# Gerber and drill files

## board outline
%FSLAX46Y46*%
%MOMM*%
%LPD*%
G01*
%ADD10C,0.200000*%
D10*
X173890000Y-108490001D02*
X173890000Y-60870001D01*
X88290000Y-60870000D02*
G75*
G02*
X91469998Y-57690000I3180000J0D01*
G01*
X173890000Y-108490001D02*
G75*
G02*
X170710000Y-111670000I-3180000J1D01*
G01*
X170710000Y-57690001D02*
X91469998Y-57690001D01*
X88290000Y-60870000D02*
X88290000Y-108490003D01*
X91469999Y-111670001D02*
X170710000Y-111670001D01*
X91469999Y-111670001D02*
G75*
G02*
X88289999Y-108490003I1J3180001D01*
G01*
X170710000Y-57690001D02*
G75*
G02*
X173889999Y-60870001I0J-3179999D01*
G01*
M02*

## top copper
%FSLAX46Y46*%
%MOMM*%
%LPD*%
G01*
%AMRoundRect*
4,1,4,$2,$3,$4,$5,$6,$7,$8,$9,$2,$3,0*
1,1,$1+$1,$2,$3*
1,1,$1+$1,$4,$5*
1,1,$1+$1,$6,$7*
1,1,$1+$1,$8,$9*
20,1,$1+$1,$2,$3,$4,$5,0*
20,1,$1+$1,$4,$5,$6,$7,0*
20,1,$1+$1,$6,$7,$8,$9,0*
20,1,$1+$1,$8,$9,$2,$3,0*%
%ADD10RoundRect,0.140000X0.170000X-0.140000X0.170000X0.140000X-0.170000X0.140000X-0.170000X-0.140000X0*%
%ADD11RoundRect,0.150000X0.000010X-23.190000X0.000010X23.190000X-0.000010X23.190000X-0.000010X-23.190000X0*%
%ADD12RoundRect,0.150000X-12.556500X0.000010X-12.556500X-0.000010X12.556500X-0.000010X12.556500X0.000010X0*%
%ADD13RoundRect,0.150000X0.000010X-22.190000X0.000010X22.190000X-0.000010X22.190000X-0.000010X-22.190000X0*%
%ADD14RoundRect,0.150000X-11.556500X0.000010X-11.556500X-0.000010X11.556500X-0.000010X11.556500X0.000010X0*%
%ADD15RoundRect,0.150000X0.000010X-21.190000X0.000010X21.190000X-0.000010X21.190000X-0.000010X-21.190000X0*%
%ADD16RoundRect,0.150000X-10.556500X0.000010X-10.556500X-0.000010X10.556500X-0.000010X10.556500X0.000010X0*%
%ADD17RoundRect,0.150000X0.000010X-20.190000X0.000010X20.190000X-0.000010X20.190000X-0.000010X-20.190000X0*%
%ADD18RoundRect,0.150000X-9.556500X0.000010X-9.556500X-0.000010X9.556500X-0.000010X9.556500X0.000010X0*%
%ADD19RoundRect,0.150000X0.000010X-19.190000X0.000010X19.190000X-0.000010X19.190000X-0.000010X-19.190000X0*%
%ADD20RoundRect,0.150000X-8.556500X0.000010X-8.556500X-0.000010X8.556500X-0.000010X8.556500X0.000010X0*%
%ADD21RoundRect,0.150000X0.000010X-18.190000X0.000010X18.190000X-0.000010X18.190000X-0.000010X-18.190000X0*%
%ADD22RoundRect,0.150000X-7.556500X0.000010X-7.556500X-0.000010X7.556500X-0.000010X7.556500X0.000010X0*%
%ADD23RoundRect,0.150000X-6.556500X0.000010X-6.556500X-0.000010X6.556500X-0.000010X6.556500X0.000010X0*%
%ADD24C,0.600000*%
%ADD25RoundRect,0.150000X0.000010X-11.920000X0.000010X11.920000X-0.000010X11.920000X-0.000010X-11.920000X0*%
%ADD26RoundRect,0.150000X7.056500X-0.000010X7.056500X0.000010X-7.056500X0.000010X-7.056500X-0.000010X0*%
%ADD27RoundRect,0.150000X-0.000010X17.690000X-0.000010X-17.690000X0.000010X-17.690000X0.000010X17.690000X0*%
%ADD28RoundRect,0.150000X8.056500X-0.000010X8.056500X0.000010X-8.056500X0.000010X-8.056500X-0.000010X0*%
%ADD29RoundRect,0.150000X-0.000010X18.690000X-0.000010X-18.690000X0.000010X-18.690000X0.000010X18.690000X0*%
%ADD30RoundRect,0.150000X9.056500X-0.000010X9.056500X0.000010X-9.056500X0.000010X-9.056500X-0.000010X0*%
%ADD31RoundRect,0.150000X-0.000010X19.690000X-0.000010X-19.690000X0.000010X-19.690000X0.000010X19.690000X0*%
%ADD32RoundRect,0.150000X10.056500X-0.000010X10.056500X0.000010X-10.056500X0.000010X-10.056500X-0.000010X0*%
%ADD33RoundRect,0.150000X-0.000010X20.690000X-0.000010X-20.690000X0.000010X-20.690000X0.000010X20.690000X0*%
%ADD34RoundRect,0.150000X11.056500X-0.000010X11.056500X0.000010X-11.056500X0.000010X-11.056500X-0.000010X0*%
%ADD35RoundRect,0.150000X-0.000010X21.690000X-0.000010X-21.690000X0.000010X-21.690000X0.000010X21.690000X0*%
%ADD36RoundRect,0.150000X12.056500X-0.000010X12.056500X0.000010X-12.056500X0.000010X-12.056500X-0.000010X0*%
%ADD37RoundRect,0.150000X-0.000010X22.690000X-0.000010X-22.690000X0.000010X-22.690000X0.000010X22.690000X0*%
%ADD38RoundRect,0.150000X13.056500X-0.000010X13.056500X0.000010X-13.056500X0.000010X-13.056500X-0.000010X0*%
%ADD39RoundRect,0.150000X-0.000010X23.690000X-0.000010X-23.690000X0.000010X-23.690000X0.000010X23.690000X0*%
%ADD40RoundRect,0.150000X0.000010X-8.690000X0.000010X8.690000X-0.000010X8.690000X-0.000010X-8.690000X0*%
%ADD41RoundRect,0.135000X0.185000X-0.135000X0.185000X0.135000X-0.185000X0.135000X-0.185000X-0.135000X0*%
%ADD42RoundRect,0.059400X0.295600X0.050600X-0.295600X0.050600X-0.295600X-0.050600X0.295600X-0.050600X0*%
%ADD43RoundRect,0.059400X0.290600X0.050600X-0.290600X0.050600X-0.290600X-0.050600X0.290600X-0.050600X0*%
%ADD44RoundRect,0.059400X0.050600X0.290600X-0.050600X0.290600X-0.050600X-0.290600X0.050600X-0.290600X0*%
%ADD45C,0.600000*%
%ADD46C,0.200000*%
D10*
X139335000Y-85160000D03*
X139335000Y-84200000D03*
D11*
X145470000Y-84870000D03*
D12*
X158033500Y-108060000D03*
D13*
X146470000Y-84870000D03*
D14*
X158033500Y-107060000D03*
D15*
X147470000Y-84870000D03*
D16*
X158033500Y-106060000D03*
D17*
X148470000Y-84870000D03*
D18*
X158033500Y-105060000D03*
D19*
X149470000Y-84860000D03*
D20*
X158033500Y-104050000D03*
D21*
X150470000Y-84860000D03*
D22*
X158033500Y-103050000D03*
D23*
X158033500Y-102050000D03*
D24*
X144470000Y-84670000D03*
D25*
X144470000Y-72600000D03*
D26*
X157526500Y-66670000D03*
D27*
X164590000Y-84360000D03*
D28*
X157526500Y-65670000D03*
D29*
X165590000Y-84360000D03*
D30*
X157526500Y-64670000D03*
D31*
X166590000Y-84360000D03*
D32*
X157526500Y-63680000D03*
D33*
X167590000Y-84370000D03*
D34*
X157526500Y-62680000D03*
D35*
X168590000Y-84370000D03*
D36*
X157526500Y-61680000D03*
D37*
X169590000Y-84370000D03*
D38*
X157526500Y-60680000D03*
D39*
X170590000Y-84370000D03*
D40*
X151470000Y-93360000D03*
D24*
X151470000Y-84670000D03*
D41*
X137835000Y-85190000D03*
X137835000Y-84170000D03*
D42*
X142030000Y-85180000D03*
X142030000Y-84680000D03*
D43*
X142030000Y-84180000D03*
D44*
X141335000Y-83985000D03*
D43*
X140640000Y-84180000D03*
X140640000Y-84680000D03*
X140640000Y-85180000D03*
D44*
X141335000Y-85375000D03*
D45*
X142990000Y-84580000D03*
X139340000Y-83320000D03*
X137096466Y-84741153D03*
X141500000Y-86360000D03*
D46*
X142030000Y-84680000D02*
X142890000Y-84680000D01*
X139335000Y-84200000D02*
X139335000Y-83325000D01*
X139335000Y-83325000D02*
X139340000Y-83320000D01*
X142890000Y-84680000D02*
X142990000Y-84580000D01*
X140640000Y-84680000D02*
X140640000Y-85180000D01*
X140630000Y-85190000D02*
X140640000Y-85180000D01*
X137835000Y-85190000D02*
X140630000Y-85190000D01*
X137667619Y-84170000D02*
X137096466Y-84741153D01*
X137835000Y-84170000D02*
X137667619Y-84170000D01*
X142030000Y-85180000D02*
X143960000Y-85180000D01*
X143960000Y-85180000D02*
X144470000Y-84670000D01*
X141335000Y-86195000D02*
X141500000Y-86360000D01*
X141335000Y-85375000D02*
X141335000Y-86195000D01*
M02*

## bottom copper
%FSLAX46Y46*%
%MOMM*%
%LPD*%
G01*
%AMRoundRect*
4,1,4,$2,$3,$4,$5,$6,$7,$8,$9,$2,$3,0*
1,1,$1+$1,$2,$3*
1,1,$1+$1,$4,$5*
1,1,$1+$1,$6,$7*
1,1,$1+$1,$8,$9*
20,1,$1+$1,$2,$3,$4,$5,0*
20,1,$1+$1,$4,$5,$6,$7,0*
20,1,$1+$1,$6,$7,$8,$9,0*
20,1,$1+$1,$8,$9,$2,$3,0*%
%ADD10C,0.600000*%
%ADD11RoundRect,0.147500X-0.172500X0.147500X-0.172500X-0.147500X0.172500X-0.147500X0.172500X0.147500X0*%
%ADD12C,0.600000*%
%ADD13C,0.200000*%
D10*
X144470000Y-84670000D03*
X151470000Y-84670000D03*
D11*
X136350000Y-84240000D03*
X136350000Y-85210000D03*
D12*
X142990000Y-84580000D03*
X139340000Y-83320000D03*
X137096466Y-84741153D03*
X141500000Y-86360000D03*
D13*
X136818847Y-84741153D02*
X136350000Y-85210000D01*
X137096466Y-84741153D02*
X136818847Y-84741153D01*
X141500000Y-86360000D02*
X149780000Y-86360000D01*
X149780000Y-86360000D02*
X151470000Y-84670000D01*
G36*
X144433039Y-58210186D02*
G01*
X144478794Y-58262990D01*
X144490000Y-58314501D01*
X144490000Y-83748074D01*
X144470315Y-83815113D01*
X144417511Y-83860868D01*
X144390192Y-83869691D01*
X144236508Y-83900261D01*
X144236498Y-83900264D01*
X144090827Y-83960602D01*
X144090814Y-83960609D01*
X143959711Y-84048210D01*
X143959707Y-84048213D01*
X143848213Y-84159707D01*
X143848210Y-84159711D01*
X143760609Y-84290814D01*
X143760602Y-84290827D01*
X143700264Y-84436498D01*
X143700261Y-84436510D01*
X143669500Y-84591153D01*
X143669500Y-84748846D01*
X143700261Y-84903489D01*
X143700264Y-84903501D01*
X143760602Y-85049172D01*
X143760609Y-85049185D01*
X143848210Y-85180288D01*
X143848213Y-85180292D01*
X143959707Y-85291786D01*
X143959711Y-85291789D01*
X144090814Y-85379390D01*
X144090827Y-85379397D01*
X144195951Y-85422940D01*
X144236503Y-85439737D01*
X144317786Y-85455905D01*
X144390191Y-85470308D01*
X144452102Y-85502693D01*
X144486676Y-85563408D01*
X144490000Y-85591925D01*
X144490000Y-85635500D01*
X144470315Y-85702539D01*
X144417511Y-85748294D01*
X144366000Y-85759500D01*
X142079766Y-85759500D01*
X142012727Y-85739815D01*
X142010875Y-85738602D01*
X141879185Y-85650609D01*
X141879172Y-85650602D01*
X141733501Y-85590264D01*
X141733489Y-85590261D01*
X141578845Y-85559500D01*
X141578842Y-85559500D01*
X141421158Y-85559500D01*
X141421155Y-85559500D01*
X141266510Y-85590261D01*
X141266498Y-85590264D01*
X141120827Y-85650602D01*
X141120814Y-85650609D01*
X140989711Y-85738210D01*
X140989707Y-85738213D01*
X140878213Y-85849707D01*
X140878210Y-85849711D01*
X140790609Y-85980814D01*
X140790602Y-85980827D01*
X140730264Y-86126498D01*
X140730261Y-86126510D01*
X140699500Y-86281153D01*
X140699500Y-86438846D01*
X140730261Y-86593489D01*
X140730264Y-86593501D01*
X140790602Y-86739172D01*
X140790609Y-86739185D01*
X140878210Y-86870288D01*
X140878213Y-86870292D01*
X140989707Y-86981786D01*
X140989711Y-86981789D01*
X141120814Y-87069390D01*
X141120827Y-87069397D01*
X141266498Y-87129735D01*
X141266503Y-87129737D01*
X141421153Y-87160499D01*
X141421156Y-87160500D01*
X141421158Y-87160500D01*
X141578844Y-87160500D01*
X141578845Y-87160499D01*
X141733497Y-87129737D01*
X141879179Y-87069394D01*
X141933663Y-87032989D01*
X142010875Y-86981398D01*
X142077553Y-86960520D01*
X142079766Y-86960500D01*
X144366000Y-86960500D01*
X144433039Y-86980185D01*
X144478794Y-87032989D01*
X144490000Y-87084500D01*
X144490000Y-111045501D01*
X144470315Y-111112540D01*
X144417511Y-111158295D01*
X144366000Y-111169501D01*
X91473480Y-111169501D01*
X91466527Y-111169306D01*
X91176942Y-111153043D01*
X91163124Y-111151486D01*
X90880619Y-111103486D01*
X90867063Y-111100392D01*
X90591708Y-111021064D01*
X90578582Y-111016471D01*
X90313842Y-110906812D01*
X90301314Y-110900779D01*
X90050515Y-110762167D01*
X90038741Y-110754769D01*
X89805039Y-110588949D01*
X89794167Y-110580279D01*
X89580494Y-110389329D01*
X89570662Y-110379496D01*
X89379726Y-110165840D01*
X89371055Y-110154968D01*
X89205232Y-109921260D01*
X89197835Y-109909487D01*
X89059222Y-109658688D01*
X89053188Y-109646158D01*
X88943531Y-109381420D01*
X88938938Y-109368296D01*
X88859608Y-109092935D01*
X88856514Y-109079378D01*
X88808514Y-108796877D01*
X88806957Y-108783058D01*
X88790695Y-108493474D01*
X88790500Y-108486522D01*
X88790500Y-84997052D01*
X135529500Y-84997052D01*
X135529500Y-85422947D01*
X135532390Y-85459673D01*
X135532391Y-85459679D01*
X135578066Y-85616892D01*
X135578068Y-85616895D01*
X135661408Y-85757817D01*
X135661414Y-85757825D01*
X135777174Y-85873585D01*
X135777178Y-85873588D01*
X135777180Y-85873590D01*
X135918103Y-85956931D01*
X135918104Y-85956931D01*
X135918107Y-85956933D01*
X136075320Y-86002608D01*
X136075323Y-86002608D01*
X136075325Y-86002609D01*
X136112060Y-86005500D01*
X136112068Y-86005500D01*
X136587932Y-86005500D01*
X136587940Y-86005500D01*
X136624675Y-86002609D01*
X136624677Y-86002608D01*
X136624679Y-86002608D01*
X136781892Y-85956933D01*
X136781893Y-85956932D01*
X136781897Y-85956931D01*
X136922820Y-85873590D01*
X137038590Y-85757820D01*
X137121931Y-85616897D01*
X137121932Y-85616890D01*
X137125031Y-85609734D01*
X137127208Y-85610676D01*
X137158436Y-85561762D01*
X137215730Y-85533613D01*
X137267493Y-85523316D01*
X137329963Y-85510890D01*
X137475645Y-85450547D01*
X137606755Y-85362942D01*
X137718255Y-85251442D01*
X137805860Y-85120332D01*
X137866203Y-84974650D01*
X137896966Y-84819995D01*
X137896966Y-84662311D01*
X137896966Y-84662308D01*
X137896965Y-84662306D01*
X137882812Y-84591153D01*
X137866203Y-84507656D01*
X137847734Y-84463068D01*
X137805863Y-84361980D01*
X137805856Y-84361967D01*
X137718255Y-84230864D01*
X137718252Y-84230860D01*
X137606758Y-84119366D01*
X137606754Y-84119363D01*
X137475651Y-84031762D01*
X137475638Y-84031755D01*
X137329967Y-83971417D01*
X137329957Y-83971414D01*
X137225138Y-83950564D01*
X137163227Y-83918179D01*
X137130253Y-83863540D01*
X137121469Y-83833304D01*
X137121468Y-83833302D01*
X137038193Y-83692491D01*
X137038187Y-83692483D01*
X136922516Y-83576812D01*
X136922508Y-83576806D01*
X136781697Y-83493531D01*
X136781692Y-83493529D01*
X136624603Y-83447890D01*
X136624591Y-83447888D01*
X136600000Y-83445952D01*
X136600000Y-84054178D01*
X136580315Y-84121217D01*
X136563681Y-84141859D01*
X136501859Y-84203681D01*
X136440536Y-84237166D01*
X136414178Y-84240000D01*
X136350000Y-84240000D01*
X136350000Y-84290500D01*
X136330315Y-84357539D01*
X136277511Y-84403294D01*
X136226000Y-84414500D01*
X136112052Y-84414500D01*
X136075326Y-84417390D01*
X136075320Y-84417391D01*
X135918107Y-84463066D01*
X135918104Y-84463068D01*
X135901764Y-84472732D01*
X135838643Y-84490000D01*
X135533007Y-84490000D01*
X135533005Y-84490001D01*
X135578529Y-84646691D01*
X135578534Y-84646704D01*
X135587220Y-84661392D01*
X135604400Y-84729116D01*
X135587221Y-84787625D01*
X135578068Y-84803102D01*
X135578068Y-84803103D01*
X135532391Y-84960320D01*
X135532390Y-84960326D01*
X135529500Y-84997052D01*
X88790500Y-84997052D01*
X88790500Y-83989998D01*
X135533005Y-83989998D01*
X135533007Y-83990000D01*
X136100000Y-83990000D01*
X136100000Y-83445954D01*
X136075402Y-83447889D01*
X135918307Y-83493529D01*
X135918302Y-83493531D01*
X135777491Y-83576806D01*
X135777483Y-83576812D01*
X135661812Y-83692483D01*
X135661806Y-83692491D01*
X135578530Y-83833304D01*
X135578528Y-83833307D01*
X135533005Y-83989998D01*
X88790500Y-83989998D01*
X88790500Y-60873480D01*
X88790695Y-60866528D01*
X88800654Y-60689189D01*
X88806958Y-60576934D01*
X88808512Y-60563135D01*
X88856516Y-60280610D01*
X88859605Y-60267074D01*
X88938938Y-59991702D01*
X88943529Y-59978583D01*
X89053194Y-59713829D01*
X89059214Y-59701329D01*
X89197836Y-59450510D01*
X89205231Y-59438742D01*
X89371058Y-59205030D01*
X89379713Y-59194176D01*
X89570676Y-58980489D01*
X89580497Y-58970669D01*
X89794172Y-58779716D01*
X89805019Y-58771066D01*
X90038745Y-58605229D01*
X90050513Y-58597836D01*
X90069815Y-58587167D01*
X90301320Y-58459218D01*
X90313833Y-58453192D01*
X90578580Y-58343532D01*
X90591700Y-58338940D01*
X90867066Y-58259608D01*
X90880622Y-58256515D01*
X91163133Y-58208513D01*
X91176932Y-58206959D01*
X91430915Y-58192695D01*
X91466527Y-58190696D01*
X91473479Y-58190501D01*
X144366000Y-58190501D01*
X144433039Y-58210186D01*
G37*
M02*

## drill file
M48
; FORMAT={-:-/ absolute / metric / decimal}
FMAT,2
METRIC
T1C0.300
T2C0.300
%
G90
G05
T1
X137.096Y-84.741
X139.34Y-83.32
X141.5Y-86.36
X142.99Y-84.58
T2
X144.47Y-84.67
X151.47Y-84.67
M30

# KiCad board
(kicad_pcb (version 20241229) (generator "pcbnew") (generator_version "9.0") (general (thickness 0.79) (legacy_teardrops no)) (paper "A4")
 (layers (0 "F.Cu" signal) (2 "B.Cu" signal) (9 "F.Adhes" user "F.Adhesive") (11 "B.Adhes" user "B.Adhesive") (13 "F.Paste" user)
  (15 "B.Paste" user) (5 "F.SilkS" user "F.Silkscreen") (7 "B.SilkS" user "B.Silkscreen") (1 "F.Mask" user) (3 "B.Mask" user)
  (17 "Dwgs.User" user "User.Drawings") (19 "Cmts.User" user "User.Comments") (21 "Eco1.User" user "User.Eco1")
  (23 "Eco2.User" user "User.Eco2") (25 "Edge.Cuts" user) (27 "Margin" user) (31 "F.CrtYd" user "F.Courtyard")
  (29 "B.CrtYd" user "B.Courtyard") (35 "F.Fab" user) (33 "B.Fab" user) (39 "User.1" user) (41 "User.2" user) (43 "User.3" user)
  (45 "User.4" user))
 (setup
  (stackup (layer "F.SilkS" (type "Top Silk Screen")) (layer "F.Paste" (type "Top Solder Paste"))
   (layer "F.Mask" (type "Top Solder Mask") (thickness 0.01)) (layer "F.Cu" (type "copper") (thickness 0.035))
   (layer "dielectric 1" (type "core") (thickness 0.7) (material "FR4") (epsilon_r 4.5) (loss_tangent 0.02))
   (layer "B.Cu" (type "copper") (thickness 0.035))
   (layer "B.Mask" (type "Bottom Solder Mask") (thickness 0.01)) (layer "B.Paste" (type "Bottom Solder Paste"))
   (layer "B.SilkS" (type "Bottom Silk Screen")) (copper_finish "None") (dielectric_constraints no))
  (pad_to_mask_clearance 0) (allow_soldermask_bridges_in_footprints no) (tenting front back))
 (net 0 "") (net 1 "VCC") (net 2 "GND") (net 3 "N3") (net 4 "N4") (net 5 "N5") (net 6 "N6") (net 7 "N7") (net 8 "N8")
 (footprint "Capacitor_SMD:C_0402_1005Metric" (layer "F.Cu") (at 139.335 84.68 90)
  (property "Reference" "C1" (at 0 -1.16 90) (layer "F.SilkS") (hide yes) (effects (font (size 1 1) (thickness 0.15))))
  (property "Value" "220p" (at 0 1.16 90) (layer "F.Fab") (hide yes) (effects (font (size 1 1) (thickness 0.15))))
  (pad "1" smd roundrect (at -0.48 0 90) (size 0.56 0.62) (layers "F.Cu" "F.Mask" "F.Paste") (roundrect_rratio 0.25) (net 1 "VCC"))
  (pad "2" smd roundrect (at 0.48 0 90) (size 0.56 0.62) (layers "F.Cu" "F.Mask" "F.Paste") (roundrect_rratio 0.25) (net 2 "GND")))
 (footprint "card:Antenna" (layer "F.Cu") (at 144.47 84.67 90)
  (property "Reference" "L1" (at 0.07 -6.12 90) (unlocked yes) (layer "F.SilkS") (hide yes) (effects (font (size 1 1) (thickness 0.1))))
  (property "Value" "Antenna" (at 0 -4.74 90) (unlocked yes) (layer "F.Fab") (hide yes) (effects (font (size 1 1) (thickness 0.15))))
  (pad "1" smd roundrect (at -23.54 1 90) (size 46.68 0.3) (drill (offset 23.34 0)) (layers "F.Cu") (roundrect_rratio 0.5) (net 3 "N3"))
  (pad "1" smd roundrect (at -23.39 26.27 270) (size 0.3 25.413) (drill (offset 0 12.7065)) (layers "F.Cu") (roundrect_rratio 0.5)
   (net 3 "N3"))
  (pad "1" smd roundrect (at -22.54 2 90) (size 44.68 0.3) (drill (offset 22.34 0)) (layers "F.Cu") (roundrect_rratio 0.5) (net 3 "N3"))
  (pad "1" smd roundrect (at -22.39 25.27 270) (size 0.3 23.413) (drill (offset 0 11.7065)) (layers "F.Cu") (roundrect_rratio 0.5)
   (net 3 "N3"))
  (pad "1" smd roundrect (at -21.54 3 90) (size 42.68 0.3) (drill (offset 21.34 0)) (layers "F.Cu") (roundrect_rratio 0.5) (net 3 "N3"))
  (pad "1" smd roundrect (at -21.39 24.27 270) (size 0.3 21.413) (drill (offset 0 10.7065)) (layers "F.Cu") (roundrect_rratio 0.5)
   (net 3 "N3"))
  (pad "1" smd roundrect (at -20.54 4 90) (size 40.68 0.3) (drill (offset 20.34 0)) (layers "F.Cu") (roundrect_rratio 0.5) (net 3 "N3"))
  (pad "1" smd roundrect (at -20.39 23.27 270) (size 0.3 19.413) (drill (offset 0 9.7065)) (layers "F.Cu") (roundrect_rratio 0.5)
   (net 3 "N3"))
  (pad "1" smd roundrect (at -19.53 5 90) (size 38.68 0.3) (drill (offset 19.34 0)) (layers "F.Cu") (roundrect_rratio 0.5) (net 3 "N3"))
  (pad "1" smd roundrect (at -19.38 22.27 270) (size 0.3 17.413) (drill (offset 0 8.7065)) (layers "F.Cu") (roundrect_rratio 0.5)
   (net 3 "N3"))
  (pad "1" smd roundrect (at -18.53 6 90) (size 36.68 0.3) (drill (offset 18.34 0)) (layers "F.Cu") (roundrect_rratio 0.5) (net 3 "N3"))
  (pad "1" smd roundrect (at -18.38 21.27 270) (size 0.3 15.413) (drill (offset 0 7.7065)) (layers "F.Cu") (roundrect_rratio 0.5)
   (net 3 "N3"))
  (pad "1" smd roundrect (at -17.38 20.27 270) (size 0.3 13.413) (drill (offset 0 6.7065)) (layers "F.Cu") (roundrect_rratio 0.5)
   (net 3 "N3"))
  (pad "1" thru_hole circle (at 0 0 270) (size 0.6 0.6) (drill 0.3) (layers "*.Cu") (remove_unused_layers no) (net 3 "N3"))
  (pad "1" smd roundrect (at 0 0 90) (size 24.14 0.3) (drill (offset 12.07 0)) (layers "F.Cu") (roundrect_rratio 0.5) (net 3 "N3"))
  (pad "1" smd roundrect (at 18 5.85 90) (size 0.3 14.413) (drill (offset 0 7.2065)) (layers "F.Cu") (roundrect_rratio 0.5) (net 3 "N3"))
  (pad "1" smd roundrect (at 18.15 20.12 270) (size 35.68 0.3) (drill (offset 17.84 0)) (layers "F.Cu") (roundrect_rratio 0.5) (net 3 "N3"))
  (pad "1" smd roundrect (at 19 4.85 90) (size 0.3 16.413) (drill (offset 0 8.2065)) (layers "F.Cu") (roundrect_rratio 0.5) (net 3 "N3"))
  (pad "1" smd roundrect (at 19.15 21.12 270) (size 37.68 0.3) (drill (offset 18.84 0)) (layers "F.Cu") (roundrect_rratio 0.5) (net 3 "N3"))
  (pad "1" smd roundrect (at 20 3.85 90) (size 0.3 18.413) (drill (offset 0 9.2065)) (layers "F.Cu") (roundrect_rratio 0.5) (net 3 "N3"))
  (pad "1" smd roundrect (at 20.15 22.12 270) (size 39.68 0.3) (drill (offset 19.84 0)) (layers "F.Cu") (roundrect_rratio 0.5) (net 3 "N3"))
  (pad "1" smd roundrect (at 20.99 2.85 90) (size 0.3 20.413) (drill (offset 0 10.2065)) (layers "F.Cu") (roundrect_rratio 0.5) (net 3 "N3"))
  (pad "1" smd roundrect (at 21.14 23.12 270) (size 41.68 0.3) (drill (offset 20.84 0)) (layers "F.Cu") (roundrect_rratio 0.5) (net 3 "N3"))
  (pad "1" smd roundrect (at 21.99 1.85 90) (size 0.3 22.413) (drill (offset 0 11.2065)) (layers "F.Cu") (roundrect_rratio 0.5) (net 3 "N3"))
  (pad "1" smd roundrect (at 22.14 24.12 270) (size 43.68 0.3) (drill (offset 21.84 0)) (layers "F.Cu") (roundrect_rratio 0.5) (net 3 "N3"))
  (pad "1" smd roundrect (at 22.99 0.85 90) (size 0.3 24.413) (drill (offset 0 12.2065)) (layers "F.Cu") (roundrect_rratio 0.5) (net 3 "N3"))
  (pad "1" smd roundrect (at 23.14 25.12 270) (size 45.68 0.3) (drill (offset 22.84 0)) (layers "F.Cu") (roundrect_rratio 0.5) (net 3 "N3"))
  (pad "1" smd roundrect (at 23.99 -0.15 90) (size 0.3 26.413) (drill (offset 0 13.2065)) (layers "F.Cu") (roundrect_rratio 0.5)
   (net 3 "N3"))
  (pad "1" smd roundrect (at 24.14 26.12 270) (size 47.68 0.3) (drill (offset 23.84 0)) (layers "F.Cu") (roundrect_rratio 0.5) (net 3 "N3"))
  (pad "2" smd roundrect (at -17.53 7 90) (size 17.68 0.3) (drill (offset 8.84 0)) (layers "F.Cu") (roundrect_rratio 0.5) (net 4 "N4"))
  (pad "2" thru_hole circle (at 0 7 270) (size 0.6 0.6) (drill 0.3) (layers "*.Cu") (remove_unused_layers no) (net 4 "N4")))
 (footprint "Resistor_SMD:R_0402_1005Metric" (layer "F.Cu") (at 137.835 84.68 90)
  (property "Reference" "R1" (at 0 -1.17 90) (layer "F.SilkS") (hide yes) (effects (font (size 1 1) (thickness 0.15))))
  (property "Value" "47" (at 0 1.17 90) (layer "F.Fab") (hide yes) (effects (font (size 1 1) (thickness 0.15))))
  (pad "1" smd roundrect (at -0.51 0 90) (size 0.54 0.64) (layers "F.Cu" "F.Mask" "F.Paste") (roundrect_rratio 0.25) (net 1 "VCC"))
  (pad "2" smd roundrect (at 0.51 0 90) (size 0.54 0.64) (layers "F.Cu" "F.Mask" "F.Paste") (roundrect_rratio 0.25) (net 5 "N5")))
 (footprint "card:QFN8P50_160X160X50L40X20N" (layer "F.Cu") (at 141.335 84.68 180)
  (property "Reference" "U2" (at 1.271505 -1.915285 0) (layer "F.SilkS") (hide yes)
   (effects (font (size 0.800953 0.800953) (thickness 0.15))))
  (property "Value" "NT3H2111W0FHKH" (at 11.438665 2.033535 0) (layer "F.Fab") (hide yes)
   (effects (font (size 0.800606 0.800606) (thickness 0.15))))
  (pad "1" smd roundrect (at -0.695 -0.5 180) (size 0.71 0.22) (layers "F.Cu" "F.Mask" "F.Paste") (roundrect_rratio 0.27) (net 3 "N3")
   (solder_mask_margin 0.102))
  (pad "2" smd roundrect (at -0.695 0 180) (size 0.71 0.22) (layers "F.Cu" "F.Mask" "F.Paste") (roundrect_rratio 0.27) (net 2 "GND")
   (solder_mask_margin 0.102))
  (pad "3" smd roundrect (at -0.695 0.5 180) (size 0.7 0.22) (layers "F.Cu" "F.Mask" "F.Paste") (roundrect_rratio 0.27) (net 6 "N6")
   (solder_mask_margin 0.102))
  (pad "4" smd roundrect (at 0 0.695 180) (size 0.22 0.7) (layers "F.Cu" "F.Mask" "F.Paste") (roundrect_rratio 0.27) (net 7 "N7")
   (solder_mask_margin 0.102))
  (pad "5" smd roundrect (at 0.695 0.5 180) (size 0.7 0.22) (layers "F.Cu" "F.Mask" "F.Paste") (roundrect_rratio 0.27) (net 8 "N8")
   (solder_mask_margin 0.102))
  (pad "6" smd roundrect (at 0.695 0 180) (size 0.7 0.22) (layers "F.Cu" "F.Mask" "F.Paste") (roundrect_rratio 0.27) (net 1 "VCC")
   (solder_mask_margin 0.102))
  (pad "7" smd roundrect (at 0.695 -0.5 180) (size 0.7 0.22) (layers "F.Cu" "F.Mask" "F.Paste") (roundrect_rratio 0.27) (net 1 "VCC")
   (solder_mask_margin 0.102))
  (pad "8" smd roundrect (at 0 -0.695 180) (size 0.22 0.7) (layers "F.Cu" "F.Mask" "F.Paste") (roundrect_rratio 0.27) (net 4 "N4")
   (solder_mask_margin 0.102)))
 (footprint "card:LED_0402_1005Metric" (layer "B.Cu") (at 136.35 84.725 -90)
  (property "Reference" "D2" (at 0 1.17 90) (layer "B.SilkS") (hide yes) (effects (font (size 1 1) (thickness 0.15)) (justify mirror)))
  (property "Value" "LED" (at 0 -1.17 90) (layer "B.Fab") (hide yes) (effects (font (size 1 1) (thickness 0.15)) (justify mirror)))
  (pad "1" smd roundrect (at -0.485 0 270) (size 0.59 0.64) (layers "B.Cu" "B.Mask" "B.Paste") (roundrect_rratio 0.25) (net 2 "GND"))
  (pad "2" smd roundrect (at 0.485 0 270) (size 0.59 0.64) (layers "B.Cu" "B.Mask" "B.Paste") (roundrect_rratio 0.25) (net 5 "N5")))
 (gr_line (start 173.89 108.490001) (end 173.89 60.870001) (stroke (width 0.2) (type solid)) (layer "Edge.Cuts"))
 (gr_arc (start 88.29 60.87) (mid 89.2214 58.621401) (end 91.469998 57.690001) (stroke (width 0.2) (type solid)) (layer "Edge.Cuts"))
 (gr_arc (start 173.89 108.490001) (mid 172.9586 110.738601) (end 170.71 111.670001) (stroke (width 0.2) (type solid)) (layer "Edge.Cuts"))
 (gr_line (start 170.71 57.690001) (end 91.469998 57.690001) (stroke (width 0.2) (type solid)) (layer "Edge.Cuts"))
 (gr_line (start 88.29 60.87) (end 88.29 108.490003) (stroke (width 0.2) (type solid)) (layer "Edge.Cuts"))
 (gr_line (start 91.469999 111.670001) (end 170.71 111.670001) (stroke (width 0.2) (type solid)) (layer "Edge.Cuts"))
 (gr_arc (start 91.469999 111.670001) (mid 89.2214 110.738601) (end 88.29 108.490003) (stroke (width 0.2) (type solid)) (layer "Edge.Cuts"))
 (gr_arc (start 170.71 57.690001) (mid 172.9586 58.621401) (end 173.89 60.870001) (stroke (width 0.2) (type solid)) (layer "Edge.Cuts"))
 (segment (start 142.03 84.68) (end 142.89 84.68) (width 0.2) (layer "F.Cu") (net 2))
 (segment (start 139.335 84.2) (end 139.335 83.325) (width 0.2) (layer "F.Cu") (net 2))
 (segment (start 139.335 83.325) (end 139.34 83.32) (width 0.2) (layer "F.Cu") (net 2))
 (segment (start 142.89 84.68) (end 142.99 84.58) (width 0.2) (layer "F.Cu") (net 2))
 (via (at 142.99 84.58) (size 0.6) (drill 0.3) (layers "F.Cu" "B.Cu") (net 2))
 (via (at 139.34 83.32) (size 0.6) (drill 0.3) (layers "F.Cu" "B.Cu") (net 2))
 (segment (start 140.64 84.68) (end 140.64 85.18) (width 0.2) (layer "F.Cu") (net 1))
 (segment (start 140.63 85.19) (end 140.64 85.18) (width 0.2) (layer "F.Cu") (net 1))
 (segment (start 137.835 85.19) (end 140.63 85.19) (width 0.2) (layer "F.Cu") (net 1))
 (segment (start 137.667619 84.17) (end 137.096466 84.741153) (width 0.2) (layer "F.Cu") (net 5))
 (segment (start 137.835 84.17) (end 137.667619 84.17) (width 0.2) (layer "F.Cu") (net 5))
 (via (at 137.096466 84.741153) (size 0.6) (drill 0.3) (layers "F.Cu" "B.Cu") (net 5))
 (segment (start 136.818847 84.741153) (end 136.35 85.21) (width 0.2) (layer "B.Cu") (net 5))
 (segment (start 137.096466 84.741153) (end 136.818847 84.741153) (width 0.2) (layer "B.Cu") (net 5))
 (segment (start 142.03 85.18) (end 143.96 85.18) (width 0.2) (layer "F.Cu") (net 3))
 (segment (start 143.96 85.18) (end 144.47 84.67) (width 0.2) (layer "F.Cu") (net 3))
 (segment (start 141.335 86.195) (end 141.5 86.36) (width 0.2) (layer "F.Cu") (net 4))
 (segment (start 141.335 85.375) (end 141.335 86.195) (width 0.2) (layer "F.Cu") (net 4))
 (via (at 141.5 86.36) (size 0.6) (drill 0.3) (layers "F.Cu" "B.Cu") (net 4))
 (segment (start 141.5 86.36) (end 149.78 86.36) (width 0.2) (layer "B.Cu") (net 4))
 (segment (start 149.78 86.36) (end 151.47 84.67) (width 0.2) (layer "B.Cu") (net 4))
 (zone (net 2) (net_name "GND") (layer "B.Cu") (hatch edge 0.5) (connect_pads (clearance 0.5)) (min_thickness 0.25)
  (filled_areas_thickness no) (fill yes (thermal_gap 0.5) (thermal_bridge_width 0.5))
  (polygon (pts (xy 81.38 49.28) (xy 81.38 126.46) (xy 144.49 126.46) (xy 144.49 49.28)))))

